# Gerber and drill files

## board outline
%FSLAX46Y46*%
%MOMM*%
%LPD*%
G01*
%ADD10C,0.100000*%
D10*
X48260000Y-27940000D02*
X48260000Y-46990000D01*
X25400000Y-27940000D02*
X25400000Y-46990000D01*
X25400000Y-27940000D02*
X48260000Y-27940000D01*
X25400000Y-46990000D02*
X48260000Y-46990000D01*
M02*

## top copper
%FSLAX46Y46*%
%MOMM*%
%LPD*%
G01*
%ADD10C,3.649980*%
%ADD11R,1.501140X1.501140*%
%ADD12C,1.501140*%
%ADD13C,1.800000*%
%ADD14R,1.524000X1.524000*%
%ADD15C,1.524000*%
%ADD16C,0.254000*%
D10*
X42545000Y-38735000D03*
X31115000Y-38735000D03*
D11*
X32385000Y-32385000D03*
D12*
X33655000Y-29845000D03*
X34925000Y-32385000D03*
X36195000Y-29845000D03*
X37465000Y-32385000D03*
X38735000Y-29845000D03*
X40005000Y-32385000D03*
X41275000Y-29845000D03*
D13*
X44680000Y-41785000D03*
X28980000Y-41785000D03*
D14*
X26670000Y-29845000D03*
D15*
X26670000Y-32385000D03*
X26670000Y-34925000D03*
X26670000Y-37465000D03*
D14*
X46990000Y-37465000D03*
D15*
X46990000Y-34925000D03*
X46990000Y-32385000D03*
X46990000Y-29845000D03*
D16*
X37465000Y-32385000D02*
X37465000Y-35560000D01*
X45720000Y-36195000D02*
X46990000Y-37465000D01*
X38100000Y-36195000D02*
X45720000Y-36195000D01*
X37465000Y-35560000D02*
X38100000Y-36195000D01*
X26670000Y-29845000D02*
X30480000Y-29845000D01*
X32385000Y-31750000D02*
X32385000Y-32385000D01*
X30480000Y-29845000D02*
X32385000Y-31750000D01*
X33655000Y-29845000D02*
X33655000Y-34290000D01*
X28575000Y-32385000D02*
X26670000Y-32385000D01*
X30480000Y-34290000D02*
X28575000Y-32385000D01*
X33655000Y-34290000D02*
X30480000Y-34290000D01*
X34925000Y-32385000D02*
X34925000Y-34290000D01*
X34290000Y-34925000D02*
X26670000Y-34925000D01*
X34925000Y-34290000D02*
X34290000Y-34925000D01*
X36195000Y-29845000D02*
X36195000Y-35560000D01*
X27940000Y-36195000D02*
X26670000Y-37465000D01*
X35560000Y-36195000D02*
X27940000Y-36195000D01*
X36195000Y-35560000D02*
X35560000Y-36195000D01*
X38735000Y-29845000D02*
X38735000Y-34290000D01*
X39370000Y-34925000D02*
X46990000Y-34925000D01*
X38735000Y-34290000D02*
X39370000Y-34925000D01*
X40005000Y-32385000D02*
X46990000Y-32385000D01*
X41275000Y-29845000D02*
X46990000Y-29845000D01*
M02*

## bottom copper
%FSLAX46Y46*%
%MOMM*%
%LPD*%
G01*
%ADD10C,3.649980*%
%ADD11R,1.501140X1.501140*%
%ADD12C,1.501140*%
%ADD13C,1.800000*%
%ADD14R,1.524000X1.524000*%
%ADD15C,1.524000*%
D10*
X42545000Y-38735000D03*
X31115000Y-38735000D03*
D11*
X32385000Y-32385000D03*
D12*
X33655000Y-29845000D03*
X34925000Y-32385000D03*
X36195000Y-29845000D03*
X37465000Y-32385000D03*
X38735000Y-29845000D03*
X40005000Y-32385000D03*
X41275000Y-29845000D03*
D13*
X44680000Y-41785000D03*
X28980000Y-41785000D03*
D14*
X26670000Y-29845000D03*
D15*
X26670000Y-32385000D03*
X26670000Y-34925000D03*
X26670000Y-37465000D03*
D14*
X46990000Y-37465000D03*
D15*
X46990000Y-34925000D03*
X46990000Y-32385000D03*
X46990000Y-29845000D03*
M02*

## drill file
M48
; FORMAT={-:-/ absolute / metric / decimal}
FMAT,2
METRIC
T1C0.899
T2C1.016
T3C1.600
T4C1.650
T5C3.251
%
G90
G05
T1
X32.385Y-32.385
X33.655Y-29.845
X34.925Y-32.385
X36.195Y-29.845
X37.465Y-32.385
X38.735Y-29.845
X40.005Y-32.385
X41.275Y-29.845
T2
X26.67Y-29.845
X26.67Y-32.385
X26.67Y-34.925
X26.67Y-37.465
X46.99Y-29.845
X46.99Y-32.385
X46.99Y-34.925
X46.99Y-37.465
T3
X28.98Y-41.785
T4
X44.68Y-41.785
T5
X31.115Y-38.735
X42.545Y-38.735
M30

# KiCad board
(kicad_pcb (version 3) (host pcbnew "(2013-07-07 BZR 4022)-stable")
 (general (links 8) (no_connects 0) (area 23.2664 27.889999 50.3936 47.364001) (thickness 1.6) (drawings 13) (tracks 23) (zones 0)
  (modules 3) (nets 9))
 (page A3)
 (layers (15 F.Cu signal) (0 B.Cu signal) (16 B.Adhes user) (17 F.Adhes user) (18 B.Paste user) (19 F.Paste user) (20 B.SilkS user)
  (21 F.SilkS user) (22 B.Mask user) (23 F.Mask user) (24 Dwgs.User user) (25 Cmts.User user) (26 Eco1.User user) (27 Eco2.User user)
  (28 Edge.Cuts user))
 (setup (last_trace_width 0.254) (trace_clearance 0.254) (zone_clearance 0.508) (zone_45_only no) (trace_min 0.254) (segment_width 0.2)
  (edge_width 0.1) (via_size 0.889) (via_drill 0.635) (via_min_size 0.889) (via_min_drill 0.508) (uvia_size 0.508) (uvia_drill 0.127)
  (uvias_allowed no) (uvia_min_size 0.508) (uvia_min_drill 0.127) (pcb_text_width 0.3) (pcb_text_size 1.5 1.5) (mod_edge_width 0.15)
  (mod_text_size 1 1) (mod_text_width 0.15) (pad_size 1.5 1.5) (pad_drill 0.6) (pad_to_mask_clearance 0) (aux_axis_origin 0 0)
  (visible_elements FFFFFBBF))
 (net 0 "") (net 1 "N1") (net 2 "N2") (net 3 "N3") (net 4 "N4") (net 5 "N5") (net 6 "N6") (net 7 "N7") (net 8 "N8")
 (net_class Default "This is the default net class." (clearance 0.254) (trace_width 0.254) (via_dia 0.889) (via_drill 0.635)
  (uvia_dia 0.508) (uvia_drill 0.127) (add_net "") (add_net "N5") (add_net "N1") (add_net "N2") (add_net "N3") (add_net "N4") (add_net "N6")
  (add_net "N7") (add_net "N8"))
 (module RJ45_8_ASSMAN (layer F.Cu) (at 36.83 38.735)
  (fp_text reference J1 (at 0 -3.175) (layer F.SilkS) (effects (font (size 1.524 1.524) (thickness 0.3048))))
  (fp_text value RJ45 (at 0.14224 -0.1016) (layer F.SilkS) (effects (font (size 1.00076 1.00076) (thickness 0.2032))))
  (pad "" thru_hole circle (at 5.715 0) (size 3.64998 3.64998) (drill 3.251199) (layers *.Cu *.Mask F.SilkS))
  (pad "" thru_hole circle (at -5.715 0) (size 3.64998 3.64998) (drill 3.251199) (layers *.Cu *.Mask F.SilkS))
  (pad 1 thru_hole rect (at -4.445 -6.35) (size 1.50114 1.50114) (drill 0.899159) (layers *.Cu *.Mask F.SilkS) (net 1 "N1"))
  (pad 2 thru_hole circle (at -3.175 -8.89) (size 1.50114 1.50114) (drill 0.899159) (layers *.Cu *.Mask F.SilkS) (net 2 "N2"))
  (pad 3 thru_hole circle (at -1.905 -6.35) (size 1.50114 1.50114) (drill 0.899159) (layers *.Cu *.Mask F.SilkS) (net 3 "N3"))
  (pad 4 thru_hole circle (at -0.635 -8.89) (size 1.50114 1.50114) (drill 0.899159) (layers *.Cu *.Mask F.SilkS) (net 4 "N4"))
  (pad 5 thru_hole circle (at 0.635 -6.35) (size 1.50114 1.50114) (drill 0.899159) (layers *.Cu *.Mask F.SilkS) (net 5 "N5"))
  (pad 6 thru_hole circle (at 1.905 -8.89) (size 1.50114 1.50114) (drill 0.899159) (layers *.Cu *.Mask F.SilkS) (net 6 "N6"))
  (pad 7 thru_hole circle (at 3.175 -6.35) (size 1.50114 1.50114) (drill 0.899159) (layers *.Cu *.Mask F.SilkS) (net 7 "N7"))
  (pad 8 thru_hole circle (at 4.445 -8.89) (size 1.50114 1.50114) (drill 0.899159) (layers *.Cu *.Mask F.SilkS) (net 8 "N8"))
  (pad "" thru_hole circle (at 7.85 3.05) (size 1.8 1.8) (drill 1.65) (layers *.Cu *.Mask F.SilkS))
  (pad "" thru_hole circle (at -7.85 3.05) (size 1.8 1.8) (drill 1.6) (layers *.Cu *.Mask F.SilkS)))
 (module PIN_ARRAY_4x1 (layer F.Cu) (at 26.67 33.655 270)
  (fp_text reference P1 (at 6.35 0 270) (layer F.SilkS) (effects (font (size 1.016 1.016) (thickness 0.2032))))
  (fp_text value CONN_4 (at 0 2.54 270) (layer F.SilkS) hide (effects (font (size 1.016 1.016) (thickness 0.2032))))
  (pad 1 thru_hole rect (at -3.81 0 270) (size 1.524 1.524) (drill 1.016) (layers *.Cu *.Mask F.SilkS) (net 1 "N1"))
  (pad 2 thru_hole circle (at -1.27 0 270) (size 1.524 1.524) (drill 1.016) (layers *.Cu *.Mask F.SilkS) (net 2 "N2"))
  (pad 3 thru_hole circle (at 1.27 0 270) (size 1.524 1.524) (drill 1.016) (layers *.Cu *.Mask F.SilkS) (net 3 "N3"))
  (pad 4 thru_hole circle (at 3.81 0 270) (size 1.524 1.524) (drill 1.016) (layers *.Cu *.Mask F.SilkS) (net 4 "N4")))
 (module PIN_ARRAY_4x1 (layer F.Cu) (at 46.99 33.655 90)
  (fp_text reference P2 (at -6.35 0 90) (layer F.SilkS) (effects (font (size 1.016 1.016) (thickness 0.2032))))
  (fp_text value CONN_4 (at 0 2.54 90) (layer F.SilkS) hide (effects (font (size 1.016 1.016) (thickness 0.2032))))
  (pad 1 thru_hole rect (at -3.81 0 90) (size 1.524 1.524) (drill 1.016) (layers *.Cu *.Mask F.SilkS) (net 5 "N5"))
  (pad 2 thru_hole circle (at -1.27 0 90) (size 1.524 1.524) (drill 1.016) (layers *.Cu *.Mask F.SilkS) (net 6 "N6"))
  (pad 3 thru_hole circle (at 1.27 0 90) (size 1.524 1.524) (drill 1.016) (layers *.Cu *.Mask F.SilkS) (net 7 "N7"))
  (pad 4 thru_hole circle (at 3.81 0 90) (size 1.524 1.524) (drill 1.016) (layers *.Cu *.Mask F.SilkS) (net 8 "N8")))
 (gr_line (start 48.26 27.94) (end 48.26 46.99) (angle 90) (layer Edge.Cuts) (width 0.1))
 (gr_line (start 25.4 27.94) (end 25.4 46.99) (angle 90) (layer Edge.Cuts) (width 0.1))
 (gr_line (start 25.4 27.94) (end 48.26 27.94) (angle 90) (layer Edge.Cuts) (width 0.1))
 (gr_line (start 25.4 46.99) (end 48.26 46.99) (angle 90) (layer Edge.Cuts) (width 0.1))
 (segment (start 37.465 32.385) (end 37.465 35.56) (width 0.254) (layer F.Cu) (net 5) (status 400000))
 (segment (start 45.72 36.195) (end 46.99 37.465) (width 0.254) (layer F.Cu) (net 5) (status 800000))
 (segment (start 38.1 36.195) (end 45.72 36.195) (width 0.254) (layer F.Cu) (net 5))
 (segment (start 37.465 35.56) (end 38.1 36.195) (width 0.254) (layer F.Cu) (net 5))
 (segment (start 26.67 29.845) (end 30.48 29.845) (width 0.254) (layer F.Cu) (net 1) (status 400000))
 (segment (start 32.385 31.75) (end 32.385 32.385) (width 0.254) (layer F.Cu) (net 1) (status C00000))
 (segment (start 30.48 29.845) (end 32.385 31.75) (width 0.254) (layer F.Cu) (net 1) (status 800000))
 (segment (start 33.655 29.845) (end 33.655 34.29) (width 0.254) (layer F.Cu) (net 2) (status 400000))
 (segment (start 28.575 32.385) (end 26.67 32.385) (width 0.254) (layer F.Cu) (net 2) (status 800000))
 (segment (start 30.48 34.29) (end 28.575 32.385) (width 0.254) (layer F.Cu) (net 2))
 (segment (start 33.655 34.29) (end 30.48 34.29) (width 0.254) (layer F.Cu) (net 2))
 (segment (start 34.925 32.385) (end 34.925 34.29) (width 0.254) (layer F.Cu) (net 3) (status 400000))
 (segment (start 34.29 34.925) (end 26.67 34.925) (width 0.254) (layer F.Cu) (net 3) (status 800000))
 (segment (start 34.925 34.29) (end 34.29 34.925) (width 0.254) (layer F.Cu) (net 3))
 (segment (start 36.195 29.845) (end 36.195 35.56) (width 0.254) (layer F.Cu) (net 4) (status 400000))
 (segment (start 27.94 36.195) (end 26.67 37.465) (width 0.254) (layer F.Cu) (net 4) (status 800000))
 (segment (start 35.56 36.195) (end 27.94 36.195) (width 0.254) (layer F.Cu) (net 4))
 (segment (start 36.195 35.56) (end 35.56 36.195) (width 0.254) (layer F.Cu) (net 4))
 (segment (start 38.735 29.845) (end 38.735 34.29) (width 0.254) (layer F.Cu) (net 6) (status 400000))
 (segment (start 39.37 34.925) (end 46.99 34.925) (width 0.254) (layer F.Cu) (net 6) (status 800000))
 (segment (start 38.735 34.29) (end 39.37 34.925) (width 0.254) (layer F.Cu) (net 6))
 (segment (start 40.005 32.385) (end 46.99 32.385) (width 0.254) (layer F.Cu) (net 7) (status C00000))
 (segment (start 41.275 29.845) (end 46.99 29.845) (width 0.254) (layer F.Cu) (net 8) (status C00000)))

